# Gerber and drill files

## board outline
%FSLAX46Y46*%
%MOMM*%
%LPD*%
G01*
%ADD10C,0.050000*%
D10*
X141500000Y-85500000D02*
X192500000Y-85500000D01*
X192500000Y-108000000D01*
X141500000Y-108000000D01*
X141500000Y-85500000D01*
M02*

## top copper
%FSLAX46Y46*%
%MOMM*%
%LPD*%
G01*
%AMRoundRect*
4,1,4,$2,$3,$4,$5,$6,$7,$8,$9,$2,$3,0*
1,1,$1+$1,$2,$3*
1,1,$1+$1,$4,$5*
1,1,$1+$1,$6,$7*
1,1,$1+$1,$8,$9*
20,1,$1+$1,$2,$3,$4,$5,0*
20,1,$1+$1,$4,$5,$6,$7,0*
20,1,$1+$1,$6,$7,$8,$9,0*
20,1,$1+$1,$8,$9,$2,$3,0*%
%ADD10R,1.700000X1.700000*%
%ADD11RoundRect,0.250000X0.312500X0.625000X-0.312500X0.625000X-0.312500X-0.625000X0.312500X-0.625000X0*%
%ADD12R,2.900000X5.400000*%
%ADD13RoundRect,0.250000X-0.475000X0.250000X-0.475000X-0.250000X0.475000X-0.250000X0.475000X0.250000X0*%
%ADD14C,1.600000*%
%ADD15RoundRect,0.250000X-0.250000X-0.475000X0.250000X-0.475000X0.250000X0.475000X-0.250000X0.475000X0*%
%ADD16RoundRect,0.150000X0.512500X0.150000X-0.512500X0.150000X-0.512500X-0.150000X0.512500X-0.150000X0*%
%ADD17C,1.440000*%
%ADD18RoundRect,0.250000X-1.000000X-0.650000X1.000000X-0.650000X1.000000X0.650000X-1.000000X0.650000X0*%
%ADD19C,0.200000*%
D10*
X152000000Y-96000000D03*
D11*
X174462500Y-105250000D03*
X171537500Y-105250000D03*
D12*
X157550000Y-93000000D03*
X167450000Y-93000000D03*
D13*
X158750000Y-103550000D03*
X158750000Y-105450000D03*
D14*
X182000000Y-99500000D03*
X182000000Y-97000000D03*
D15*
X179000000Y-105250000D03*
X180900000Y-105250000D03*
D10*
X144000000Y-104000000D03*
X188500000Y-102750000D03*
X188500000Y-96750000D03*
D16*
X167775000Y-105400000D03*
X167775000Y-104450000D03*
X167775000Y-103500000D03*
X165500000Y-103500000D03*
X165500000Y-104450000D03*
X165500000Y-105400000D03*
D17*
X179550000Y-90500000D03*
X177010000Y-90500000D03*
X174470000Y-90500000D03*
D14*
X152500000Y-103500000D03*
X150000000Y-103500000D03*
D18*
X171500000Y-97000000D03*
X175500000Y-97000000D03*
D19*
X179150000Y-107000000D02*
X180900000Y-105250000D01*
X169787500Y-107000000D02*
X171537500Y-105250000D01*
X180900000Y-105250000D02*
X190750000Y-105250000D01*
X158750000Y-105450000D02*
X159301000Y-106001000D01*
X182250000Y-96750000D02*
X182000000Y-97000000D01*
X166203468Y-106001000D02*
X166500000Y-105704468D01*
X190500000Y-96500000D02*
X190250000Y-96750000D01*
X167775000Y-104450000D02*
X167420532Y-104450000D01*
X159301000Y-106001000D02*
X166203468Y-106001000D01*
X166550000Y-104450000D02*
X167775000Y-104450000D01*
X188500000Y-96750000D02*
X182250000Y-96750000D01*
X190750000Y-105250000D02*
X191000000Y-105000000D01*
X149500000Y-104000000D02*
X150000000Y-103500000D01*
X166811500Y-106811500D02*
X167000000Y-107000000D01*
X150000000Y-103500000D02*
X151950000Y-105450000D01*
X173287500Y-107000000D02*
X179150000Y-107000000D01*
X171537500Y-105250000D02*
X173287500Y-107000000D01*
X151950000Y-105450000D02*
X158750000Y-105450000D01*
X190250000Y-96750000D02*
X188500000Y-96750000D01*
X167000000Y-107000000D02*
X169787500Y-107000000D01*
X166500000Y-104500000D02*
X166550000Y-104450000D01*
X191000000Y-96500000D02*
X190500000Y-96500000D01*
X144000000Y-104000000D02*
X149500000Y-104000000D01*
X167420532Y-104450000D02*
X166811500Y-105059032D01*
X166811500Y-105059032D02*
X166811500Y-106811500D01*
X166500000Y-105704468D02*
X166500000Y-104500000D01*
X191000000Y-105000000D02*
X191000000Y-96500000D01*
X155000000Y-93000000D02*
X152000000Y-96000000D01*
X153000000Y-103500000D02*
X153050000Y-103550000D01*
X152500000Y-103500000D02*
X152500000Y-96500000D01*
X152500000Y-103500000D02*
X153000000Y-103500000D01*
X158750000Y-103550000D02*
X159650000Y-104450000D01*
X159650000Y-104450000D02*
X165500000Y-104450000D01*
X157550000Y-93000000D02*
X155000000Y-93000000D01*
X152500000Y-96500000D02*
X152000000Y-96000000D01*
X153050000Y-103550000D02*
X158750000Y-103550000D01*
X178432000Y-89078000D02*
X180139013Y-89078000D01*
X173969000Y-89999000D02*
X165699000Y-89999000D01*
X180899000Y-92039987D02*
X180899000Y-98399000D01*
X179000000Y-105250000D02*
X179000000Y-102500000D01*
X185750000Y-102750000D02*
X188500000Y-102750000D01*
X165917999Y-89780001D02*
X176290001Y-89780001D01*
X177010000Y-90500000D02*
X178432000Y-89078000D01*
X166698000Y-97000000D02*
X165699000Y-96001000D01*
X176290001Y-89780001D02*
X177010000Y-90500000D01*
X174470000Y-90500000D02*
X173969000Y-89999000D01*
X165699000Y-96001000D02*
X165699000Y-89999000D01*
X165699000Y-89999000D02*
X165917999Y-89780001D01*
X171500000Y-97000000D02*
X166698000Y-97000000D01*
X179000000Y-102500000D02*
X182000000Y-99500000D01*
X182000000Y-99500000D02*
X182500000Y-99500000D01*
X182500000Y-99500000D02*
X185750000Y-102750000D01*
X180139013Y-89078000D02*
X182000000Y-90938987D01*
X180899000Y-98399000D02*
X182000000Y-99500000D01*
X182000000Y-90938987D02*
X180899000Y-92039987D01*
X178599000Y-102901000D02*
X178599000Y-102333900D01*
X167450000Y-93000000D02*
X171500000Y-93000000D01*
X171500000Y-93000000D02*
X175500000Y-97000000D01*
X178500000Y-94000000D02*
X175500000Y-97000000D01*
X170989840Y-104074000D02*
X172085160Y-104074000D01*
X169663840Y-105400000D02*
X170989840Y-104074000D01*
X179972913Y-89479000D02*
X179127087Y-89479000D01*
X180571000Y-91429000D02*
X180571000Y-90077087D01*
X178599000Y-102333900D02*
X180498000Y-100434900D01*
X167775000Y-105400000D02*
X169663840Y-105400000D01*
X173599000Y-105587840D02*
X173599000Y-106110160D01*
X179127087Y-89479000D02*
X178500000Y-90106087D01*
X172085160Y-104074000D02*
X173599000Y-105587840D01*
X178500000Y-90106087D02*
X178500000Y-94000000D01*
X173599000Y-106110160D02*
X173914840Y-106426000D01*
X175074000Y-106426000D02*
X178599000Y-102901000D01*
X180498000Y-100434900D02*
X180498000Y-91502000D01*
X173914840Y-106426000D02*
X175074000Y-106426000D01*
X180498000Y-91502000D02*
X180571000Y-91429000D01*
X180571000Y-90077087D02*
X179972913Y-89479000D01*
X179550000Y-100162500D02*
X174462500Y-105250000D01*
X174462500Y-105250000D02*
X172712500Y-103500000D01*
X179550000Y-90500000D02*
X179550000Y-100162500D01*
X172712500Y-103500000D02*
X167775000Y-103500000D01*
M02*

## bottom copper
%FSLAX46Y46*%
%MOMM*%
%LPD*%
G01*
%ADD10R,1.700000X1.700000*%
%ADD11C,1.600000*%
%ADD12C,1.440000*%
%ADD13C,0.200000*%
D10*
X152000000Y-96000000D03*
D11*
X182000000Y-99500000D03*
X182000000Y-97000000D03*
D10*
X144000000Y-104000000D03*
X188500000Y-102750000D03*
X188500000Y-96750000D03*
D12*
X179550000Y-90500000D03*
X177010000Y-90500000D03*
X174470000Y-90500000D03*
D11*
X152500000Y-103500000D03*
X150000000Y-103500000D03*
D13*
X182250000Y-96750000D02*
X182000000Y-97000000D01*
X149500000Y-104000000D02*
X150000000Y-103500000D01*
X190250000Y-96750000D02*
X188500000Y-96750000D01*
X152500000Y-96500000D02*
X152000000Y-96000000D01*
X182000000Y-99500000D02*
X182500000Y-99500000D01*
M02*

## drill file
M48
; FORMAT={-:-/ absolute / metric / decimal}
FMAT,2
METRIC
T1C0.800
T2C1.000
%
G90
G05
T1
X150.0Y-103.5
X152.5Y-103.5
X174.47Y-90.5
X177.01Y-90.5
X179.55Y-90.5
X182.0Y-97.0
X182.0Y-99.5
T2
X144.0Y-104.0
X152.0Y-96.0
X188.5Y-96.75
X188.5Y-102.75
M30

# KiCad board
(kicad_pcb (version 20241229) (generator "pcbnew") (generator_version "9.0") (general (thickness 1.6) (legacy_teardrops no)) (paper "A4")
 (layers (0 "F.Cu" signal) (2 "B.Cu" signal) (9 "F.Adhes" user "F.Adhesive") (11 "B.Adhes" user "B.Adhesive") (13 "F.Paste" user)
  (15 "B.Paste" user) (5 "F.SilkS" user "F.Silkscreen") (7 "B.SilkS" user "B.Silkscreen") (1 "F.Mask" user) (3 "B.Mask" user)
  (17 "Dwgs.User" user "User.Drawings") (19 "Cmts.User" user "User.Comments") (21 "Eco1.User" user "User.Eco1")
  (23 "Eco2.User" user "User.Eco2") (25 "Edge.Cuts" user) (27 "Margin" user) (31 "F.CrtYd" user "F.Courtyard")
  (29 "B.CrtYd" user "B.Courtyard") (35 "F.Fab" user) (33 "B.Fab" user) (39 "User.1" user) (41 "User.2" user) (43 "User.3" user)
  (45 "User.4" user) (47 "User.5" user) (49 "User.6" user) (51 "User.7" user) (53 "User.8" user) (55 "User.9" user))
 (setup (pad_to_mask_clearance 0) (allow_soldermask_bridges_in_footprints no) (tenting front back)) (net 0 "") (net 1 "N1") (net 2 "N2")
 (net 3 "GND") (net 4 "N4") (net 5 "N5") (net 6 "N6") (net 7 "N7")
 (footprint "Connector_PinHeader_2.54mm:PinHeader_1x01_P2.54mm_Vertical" (layer "F.Cu") (at 152 96)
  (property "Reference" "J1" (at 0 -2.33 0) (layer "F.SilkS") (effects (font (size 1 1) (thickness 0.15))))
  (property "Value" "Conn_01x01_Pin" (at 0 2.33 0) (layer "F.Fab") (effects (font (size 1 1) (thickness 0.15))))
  (pad "1" thru_hole rect (at 0 0) (size 1.7 1.7) (drill 1) (layers "*.Cu" "*.Mask") (remove_unused_layers no) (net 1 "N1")))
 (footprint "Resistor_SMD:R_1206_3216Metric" (layer "F.Cu") (at 173 105.25 180)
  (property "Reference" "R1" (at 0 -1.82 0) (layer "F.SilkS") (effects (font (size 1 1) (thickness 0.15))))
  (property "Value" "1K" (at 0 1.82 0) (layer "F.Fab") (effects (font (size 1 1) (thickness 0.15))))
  (pad "1" smd roundrect (at -1.4625 0 180) (size 1.125 1.75) (layers "F.Cu" "F.Mask" "F.Paste") (roundrect_rratio 0.222222) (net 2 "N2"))
  (pad "2" smd roundrect (at 1.4625 0 180) (size 1.125 1.75) (layers "F.Cu" "F.Mask" "F.Paste") (roundrect_rratio 0.222222) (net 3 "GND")))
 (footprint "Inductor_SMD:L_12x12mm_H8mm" (layer "F.Cu") (at 162.5 93)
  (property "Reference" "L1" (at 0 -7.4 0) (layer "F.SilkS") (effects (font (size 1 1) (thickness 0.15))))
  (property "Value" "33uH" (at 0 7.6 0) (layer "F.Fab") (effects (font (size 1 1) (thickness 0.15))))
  (pad "1" smd rect (at -4.95 0) (size 2.9 5.4) (layers "F.Cu" "F.Mask" "F.Paste") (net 1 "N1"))
  (pad "2" smd rect (at 4.95 0) (size 2.9 5.4) (layers "F.Cu" "F.Mask" "F.Paste") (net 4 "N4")))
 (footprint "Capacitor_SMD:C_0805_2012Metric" (layer "F.Cu") (at 158.75 104.5 -90)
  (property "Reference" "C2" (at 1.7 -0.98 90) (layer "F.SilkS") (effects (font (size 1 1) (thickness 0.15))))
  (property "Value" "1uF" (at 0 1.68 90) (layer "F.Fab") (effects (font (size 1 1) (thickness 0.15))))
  (pad "1" smd roundrect (at -0.95 0 270) (size 1 1.45) (layers "F.Cu" "F.Mask" "F.Paste") (roundrect_rratio 0.25) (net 1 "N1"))
  (pad "2" smd roundrect (at 0.95 0 270) (size 1 1.45) (layers "F.Cu" "F.Mask" "F.Paste") (roundrect_rratio 0.25) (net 3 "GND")))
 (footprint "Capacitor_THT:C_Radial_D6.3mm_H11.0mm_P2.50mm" (layer "F.Cu") (at 182 99.5 90)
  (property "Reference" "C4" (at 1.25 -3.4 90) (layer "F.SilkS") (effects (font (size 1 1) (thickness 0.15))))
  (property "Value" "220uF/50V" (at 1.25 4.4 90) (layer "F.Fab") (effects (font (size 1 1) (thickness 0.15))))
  (pad "1" thru_hole circle (at 0 0 90) (size 1.6 1.6) (drill 0.8) (layers "*.Cu" "*.Mask") (remove_unused_layers no) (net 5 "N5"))
  (pad "2" thru_hole circle (at 2.5 0 90) (size 1.6 1.6) (drill 0.8) (layers "*.Cu" "*.Mask") (remove_unused_layers no) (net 3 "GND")))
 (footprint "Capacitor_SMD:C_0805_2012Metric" (layer "F.Cu") (at 179.95 105.25)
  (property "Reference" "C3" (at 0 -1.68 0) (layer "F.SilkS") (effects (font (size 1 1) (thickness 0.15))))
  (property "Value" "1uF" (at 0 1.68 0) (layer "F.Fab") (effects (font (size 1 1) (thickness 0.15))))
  (pad "1" smd roundrect (at -0.95 0) (size 1 1.45) (layers "F.Cu" "F.Mask" "F.Paste") (roundrect_rratio 0.25) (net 5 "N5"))
  (pad "2" smd roundrect (at 0.95 0) (size 1 1.45) (layers "F.Cu" "F.Mask" "F.Paste") (roundrect_rratio 0.25) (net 3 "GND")))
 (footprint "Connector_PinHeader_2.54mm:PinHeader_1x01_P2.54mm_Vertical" (layer "F.Cu") (at 144 104)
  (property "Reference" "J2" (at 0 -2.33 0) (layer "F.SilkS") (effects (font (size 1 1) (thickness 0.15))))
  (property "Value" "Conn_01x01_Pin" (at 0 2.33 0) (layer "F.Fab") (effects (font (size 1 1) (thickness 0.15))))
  (pad "1" thru_hole rect (at 0 0) (size 1.7 1.7) (drill 1) (layers "*.Cu" "*.Mask") (remove_unused_layers no) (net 3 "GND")))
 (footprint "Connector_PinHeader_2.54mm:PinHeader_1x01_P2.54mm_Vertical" (layer "F.Cu") (at 188.5 102.75)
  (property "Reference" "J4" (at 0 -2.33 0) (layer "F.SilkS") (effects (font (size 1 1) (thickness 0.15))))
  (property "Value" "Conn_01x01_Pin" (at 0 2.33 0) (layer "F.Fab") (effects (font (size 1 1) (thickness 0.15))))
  (pad "1" thru_hole rect (at 0 0) (size 1.7 1.7) (drill 1) (layers "*.Cu" "*.Mask") (remove_unused_layers no) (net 5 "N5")))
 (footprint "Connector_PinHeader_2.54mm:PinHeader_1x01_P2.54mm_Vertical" (layer "F.Cu") (at 188.5 96.75)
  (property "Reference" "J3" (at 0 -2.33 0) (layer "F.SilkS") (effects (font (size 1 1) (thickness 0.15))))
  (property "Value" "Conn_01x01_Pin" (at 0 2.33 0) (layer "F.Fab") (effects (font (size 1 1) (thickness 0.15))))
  (pad "1" thru_hole rect (at 0 0) (size 1.7 1.7) (drill 1) (layers "*.Cu" "*.Mask") (remove_unused_layers no) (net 3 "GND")))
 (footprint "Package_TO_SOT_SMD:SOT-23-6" (layer "F.Cu") (at 166.6375 104.45 180)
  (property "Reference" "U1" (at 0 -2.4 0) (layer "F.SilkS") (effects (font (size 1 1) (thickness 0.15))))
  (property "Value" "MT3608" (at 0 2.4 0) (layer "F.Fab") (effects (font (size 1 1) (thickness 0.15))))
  (pad "1" smd roundrect (at -1.1375 -0.95 180) (size 1.325 0.6) (layers "F.Cu" "F.Mask" "F.Paste") (roundrect_rratio 0.25) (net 4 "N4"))
  (pad "2" smd roundrect (at -1.1375 0 180) (size 1.325 0.6) (layers "F.Cu" "F.Mask" "F.Paste") (roundrect_rratio 0.25) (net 3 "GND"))
  (pad "3" smd roundrect (at -1.1375 0.95 180) (size 1.325 0.6) (layers "F.Cu" "F.Mask" "F.Paste") (roundrect_rratio 0.25) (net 2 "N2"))
  (pad "4" smd roundrect (at 1.1375 0.95 180) (size 1.325 0.6) (layers "F.Cu" "F.Mask" "F.Paste") (roundrect_rratio 0.25) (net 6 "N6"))
  (pad "5" smd roundrect (at 1.1375 0 180) (size 1.325 0.6) (layers "F.Cu" "F.Mask" "F.Paste") (roundrect_rratio 0.25) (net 1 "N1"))
  (pad "6" smd roundrect (at 1.1375 -0.95 180) (size 1.325 0.6) (layers "F.Cu" "F.Mask" "F.Paste") (roundrect_rratio 0.25) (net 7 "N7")))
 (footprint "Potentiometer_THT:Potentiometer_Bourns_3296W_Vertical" (layer "F.Cu") (at 179.55 90.5)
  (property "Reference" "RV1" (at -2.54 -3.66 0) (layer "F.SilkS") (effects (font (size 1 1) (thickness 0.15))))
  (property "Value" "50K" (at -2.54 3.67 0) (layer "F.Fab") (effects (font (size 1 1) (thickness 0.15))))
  (pad "1" thru_hole circle (at 0 0) (size 1.44 1.44) (drill 0.8) (layers "*.Cu" "*.Mask") (remove_unused_layers no) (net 2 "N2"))
  (pad "2" thru_hole circle (at -2.54 0) (size 1.44 1.44) (drill 0.8) (layers "*.Cu" "*.Mask") (remove_unused_layers no) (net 5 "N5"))
  (pad "3" thru_hole circle (at -5.08 0) (size 1.44 1.44) (drill 0.8) (layers "*.Cu" "*.Mask") (remove_unused_layers no) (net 5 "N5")))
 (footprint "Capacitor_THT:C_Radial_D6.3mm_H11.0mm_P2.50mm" (layer "F.Cu") (at 152.5 103.5 180)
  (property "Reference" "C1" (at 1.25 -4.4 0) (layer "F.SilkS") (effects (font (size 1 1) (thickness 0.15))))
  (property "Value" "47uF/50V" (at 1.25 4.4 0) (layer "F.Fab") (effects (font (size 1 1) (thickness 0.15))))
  (pad "1" thru_hole circle (at 0 0 180) (size 1.6 1.6) (drill 0.8) (layers "*.Cu" "*.Mask") (remove_unused_layers no) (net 1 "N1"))
  (pad "2" thru_hole circle (at 2.5 0 180) (size 1.6 1.6) (drill 0.8) (layers "*.Cu" "*.Mask") (remove_unused_layers no) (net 3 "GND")))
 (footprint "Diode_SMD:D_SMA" (layer "F.Cu") (at 173.5 97)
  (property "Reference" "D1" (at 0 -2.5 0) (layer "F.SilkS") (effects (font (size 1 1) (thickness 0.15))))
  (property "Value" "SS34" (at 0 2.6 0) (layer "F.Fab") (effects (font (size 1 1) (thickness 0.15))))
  (pad "1" smd roundrect (at -2 0) (size 2.5 1.8) (layers "F.Cu" "F.Mask" "F.Paste") (roundrect_rratio 0.1388888889) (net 5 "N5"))
  (pad "2" smd roundrect (at 2 0) (size 2.5 1.8) (layers "F.Cu" "F.Mask" "F.Paste") (roundrect_rratio 0.1388888889) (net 4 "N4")))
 (gr_rect (start 141.5 85.5) (end 192.5 108) (stroke (width 0.05) (type default)) (fill no) (layer "Edge.Cuts"))
 (segment (start 179.15 107) (end 180.9 105.25) (width 0.2) (layer "F.Cu") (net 3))
 (segment (start 169.7875 107) (end 171.5375 105.25) (width 0.2) (layer "F.Cu") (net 3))
 (segment (start 180.9 105.25) (end 190.75 105.25) (width 0.2) (layer "F.Cu") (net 3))
 (segment (start 158.75 105.45) (end 159.301 106.001) (width 0.2) (layer "F.Cu") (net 3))
 (segment (start 182.25 96.75) (end 182 97) (width 0.2) (layer "F.Cu") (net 3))
 (segment (start 166.203468 106.001) (end 166.5 105.704468) (width 0.2) (layer "F.Cu") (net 3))
 (segment (start 190.5 96.5) (end 190.25 96.75) (width 0.2) (layer "F.Cu") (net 3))
 (segment (start 167.775 104.45) (end 167.420532 104.45) (width 0.2) (layer "F.Cu") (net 3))
 (segment (start 159.301 106.001) (end 166.203468 106.001) (width 0.2) (layer "F.Cu") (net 3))
 (segment (start 166.55 104.45) (end 167.775 104.45) (width 0.2) (layer "F.Cu") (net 3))
 (segment (start 188.5 96.75) (end 182.25 96.75) (width 0.2) (layer "F.Cu") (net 3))
 (segment (start 190.75 105.25) (end 191 105) (width 0.2) (layer "F.Cu") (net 3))
 (segment (start 149.5 104) (end 150 103.5) (width 0.2) (layer "F.Cu") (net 3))
 (segment (start 166.8115 106.8115) (end 167 107) (width 0.2) (layer "F.Cu") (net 3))
 (segment (start 150 103.5) (end 151.95 105.45) (width 0.2) (layer "F.Cu") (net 3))
 (segment (start 173.2875 107) (end 179.15 107) (width 0.2) (layer "F.Cu") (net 3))
 (segment (start 171.5375 105.25) (end 173.2875 107) (width 0.2) (layer "F.Cu") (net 3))
 (segment (start 151.95 105.45) (end 158.75 105.45) (width 0.2) (layer "F.Cu") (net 3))
 (segment (start 190.25 96.75) (end 188.5 96.75) (width 0.2) (layer "F.Cu") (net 3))
 (segment (start 167 107) (end 169.7875 107) (width 0.2) (layer "F.Cu") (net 3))
 (segment (start 166.5 104.5) (end 166.55 104.45) (width 0.2) (layer "F.Cu") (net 3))
 (segment (start 191 96.5) (end 190.5 96.5) (width 0.2) (layer "F.Cu") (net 3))
 (segment (start 144 104) (end 149.5 104) (width 0.2) (layer "F.Cu") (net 3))
 (segment (start 167.420532 104.45) (end 166.8115 105.059032) (width 0.2) (layer "F.Cu") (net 3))
 (segment (start 166.8115 105.059032) (end 166.8115 106.8115) (width 0.2) (layer "F.Cu") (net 3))
 (segment (start 166.5 105.704468) (end 166.5 104.5) (width 0.2) (layer "F.Cu") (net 3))
 (segment (start 191 105) (end 191 96.5) (width 0.2) (layer "F.Cu") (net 3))
 (segment (start 182.25 96.75) (end 182 97) (width 0.2) (layer "B.Cu") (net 3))
 (segment (start 149.5 104) (end 150 103.5) (width 0.2) (layer "B.Cu") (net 3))
 (segment (start 190.25 96.75) (end 188.5 96.75) (width 0.2) (layer "B.Cu") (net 3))
 (segment (start 155 93) (end 152 96) (width 0.2) (layer "F.Cu") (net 1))
 (segment (start 153 103.5) (end 153.05 103.55) (width 0.2) (layer "F.Cu") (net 1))
 (segment (start 152.5 103.5) (end 152.5 96.5) (width 0.2) (layer "F.Cu") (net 1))
 (segment (start 152.5 103.5) (end 153 103.5) (width 0.2) (layer "F.Cu") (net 1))
 (segment (start 158.75 103.55) (end 159.65 104.45) (width 0.2) (layer "F.Cu") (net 1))
 (segment (start 159.65 104.45) (end 165.5 104.45) (width 0.2) (layer "F.Cu") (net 1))
 (segment (start 157.55 93) (end 155 93) (width 0.2) (layer "F.Cu") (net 1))
 (segment (start 152.5 96.5) (end 152 96) (width 0.2) (layer "F.Cu") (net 1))
 (segment (start 153.05 103.55) (end 158.75 103.55) (width 0.2) (layer "F.Cu") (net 1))
 (segment (start 152.5 96.5) (end 152 96) (width 0.2) (layer "B.Cu") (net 1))
 (segment (start 178.432 89.078) (end 180.139013 89.078) (width 0.2) (layer "F.Cu") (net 5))
 (segment (start 173.969 89.999) (end 165.699 89.999) (width 0.2) (layer "F.Cu") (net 5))
 (segment (start 180.899 92.039987) (end 180.899 98.399) (width 0.2) (layer "F.Cu") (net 5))
 (segment (start 179 105.25) (end 179 102.5) (width 0.2) (layer "F.Cu") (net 5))
 (segment (start 185.75 102.75) (end 188.5 102.75) (width 0.2) (layer "F.Cu") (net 5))
 (segment (start 165.917999 89.780001) (end 176.290001 89.780001) (width 0.2) (layer "F.Cu") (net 5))
 (segment (start 177.01 90.5) (end 178.432 89.078) (width 0.2) (layer "F.Cu") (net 5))
 (segment (start 166.698 97) (end 165.699 96.001) (width 0.2) (layer "F.Cu") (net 5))
 (segment (start 176.290001 89.780001) (end 177.01 90.5) (width 0.2) (layer "F.Cu") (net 5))
 (segment (start 174.47 90.5) (end 173.969 89.999) (width 0.2) (layer "F.Cu") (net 5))
 (segment (start 165.699 96.001) (end 165.699 89.999) (width 0.2) (layer "F.Cu") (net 5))
 (segment (start 165.699 89.999) (end 165.917999 89.780001) (width 0.2) (layer "F.Cu") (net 5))
 (segment (start 171.5 97) (end 166.698 97) (width 0.2) (layer "F.Cu") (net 5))
 (segment (start 179 102.5) (end 182 99.5) (width 0.2) (layer "F.Cu") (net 5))
 (segment (start 182 99.5) (end 182.5 99.5) (width 0.2) (layer "F.Cu") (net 5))
 (segment (start 182.5 99.5) (end 185.75 102.75) (width 0.2) (layer "F.Cu") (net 5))
 (segment (start 180.139013 89.078) (end 182 90.938987) (width 0.2) (layer "F.Cu") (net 5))
 (segment (start 180.899 98.399) (end 182 99.5) (width 0.2) (layer "F.Cu") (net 5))
 (segment (start 182 90.938987) (end 180.899 92.039987) (width 0.2) (layer "F.Cu") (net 5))
 (segment (start 182 99.5) (end 182.5 99.5) (width 0.2) (layer "B.Cu") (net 5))
 (segment (start 178.599 102.901) (end 178.599 102.3339) (width 0.2) (layer "F.Cu") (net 4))
 (segment (start 167.45 93) (end 171.5 93) (width 0.2) (layer "F.Cu") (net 4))
 (segment (start 171.5 93) (end 175.5 97) (width 0.2) (layer "F.Cu") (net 4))
 (segment (start 178.5 94) (end 175.5 97) (width 0.2) (layer "F.Cu") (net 4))
 (segment (start 170.98984 104.074) (end 172.08516 104.074) (width 0.2) (layer "F.Cu") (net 4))
 (segment (start 169.66384 105.4) (end 170.98984 104.074) (width 0.2) (layer "F.Cu") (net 4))
 (segment (start 179.972913 89.479) (end 179.127087 89.479) (width 0.2) (layer "F.Cu") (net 4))
 (segment (start 180.571 91.429) (end 180.571 90.077087) (width 0.2) (layer "F.Cu") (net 4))
 (segment (start 178.599 102.3339) (end 180.498 100.4349) (width 0.2) (layer "F.Cu") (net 4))
 (segment (start 167.775 105.4) (end 169.66384 105.4) (width 0.2) (layer "F.Cu") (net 4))
 (segment (start 173.599 105.58784) (end 173.599 106.11016) (width 0.2) (layer "F.Cu") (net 4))
 (segment (start 179.127087 89.479) (end 178.5 90.106087) (width 0.2) (layer "F.Cu") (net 4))
 (segment (start 172.08516 104.074) (end 173.599 105.58784) (width 0.2) (layer "F.Cu") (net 4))
 (segment (start 178.5 90.106087) (end 178.5 94) (width 0.2) (layer "F.Cu") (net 4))
 (segment (start 173.599 106.11016) (end 173.91484 106.426) (width 0.2) (layer "F.Cu") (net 4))
 (segment (start 175.074 106.426) (end 178.599 102.901) (width 0.2) (layer "F.Cu") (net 4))
 (segment (start 180.498 100.4349) (end 180.498 91.502) (width 0.2) (layer "F.Cu") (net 4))
 (segment (start 173.91484 106.426) (end 175.074 106.426) (width 0.2) (layer "F.Cu") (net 4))
 (segment (start 180.498 91.502) (end 180.571 91.429) (width 0.2) (layer "F.Cu") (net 4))
 (segment (start 180.571 90.077087) (end 179.972913 89.479) (width 0.2) (layer "F.Cu") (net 4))
 (segment (start 179.55 100.1625) (end 174.4625 105.25) (width 0.2) (layer "F.Cu") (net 2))
 (segment (start 174.4625 105.25) (end 172.7125 103.5) (width 0.2) (layer "F.Cu") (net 2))
 (segment (start 179.55 90.5) (end 179.55 100.1625) (width 0.2) (layer "F.Cu") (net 2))
 (segment (start 172.7125 103.5) (end 167.775 103.5) (width 0.2) (layer "F.Cu") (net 2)))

